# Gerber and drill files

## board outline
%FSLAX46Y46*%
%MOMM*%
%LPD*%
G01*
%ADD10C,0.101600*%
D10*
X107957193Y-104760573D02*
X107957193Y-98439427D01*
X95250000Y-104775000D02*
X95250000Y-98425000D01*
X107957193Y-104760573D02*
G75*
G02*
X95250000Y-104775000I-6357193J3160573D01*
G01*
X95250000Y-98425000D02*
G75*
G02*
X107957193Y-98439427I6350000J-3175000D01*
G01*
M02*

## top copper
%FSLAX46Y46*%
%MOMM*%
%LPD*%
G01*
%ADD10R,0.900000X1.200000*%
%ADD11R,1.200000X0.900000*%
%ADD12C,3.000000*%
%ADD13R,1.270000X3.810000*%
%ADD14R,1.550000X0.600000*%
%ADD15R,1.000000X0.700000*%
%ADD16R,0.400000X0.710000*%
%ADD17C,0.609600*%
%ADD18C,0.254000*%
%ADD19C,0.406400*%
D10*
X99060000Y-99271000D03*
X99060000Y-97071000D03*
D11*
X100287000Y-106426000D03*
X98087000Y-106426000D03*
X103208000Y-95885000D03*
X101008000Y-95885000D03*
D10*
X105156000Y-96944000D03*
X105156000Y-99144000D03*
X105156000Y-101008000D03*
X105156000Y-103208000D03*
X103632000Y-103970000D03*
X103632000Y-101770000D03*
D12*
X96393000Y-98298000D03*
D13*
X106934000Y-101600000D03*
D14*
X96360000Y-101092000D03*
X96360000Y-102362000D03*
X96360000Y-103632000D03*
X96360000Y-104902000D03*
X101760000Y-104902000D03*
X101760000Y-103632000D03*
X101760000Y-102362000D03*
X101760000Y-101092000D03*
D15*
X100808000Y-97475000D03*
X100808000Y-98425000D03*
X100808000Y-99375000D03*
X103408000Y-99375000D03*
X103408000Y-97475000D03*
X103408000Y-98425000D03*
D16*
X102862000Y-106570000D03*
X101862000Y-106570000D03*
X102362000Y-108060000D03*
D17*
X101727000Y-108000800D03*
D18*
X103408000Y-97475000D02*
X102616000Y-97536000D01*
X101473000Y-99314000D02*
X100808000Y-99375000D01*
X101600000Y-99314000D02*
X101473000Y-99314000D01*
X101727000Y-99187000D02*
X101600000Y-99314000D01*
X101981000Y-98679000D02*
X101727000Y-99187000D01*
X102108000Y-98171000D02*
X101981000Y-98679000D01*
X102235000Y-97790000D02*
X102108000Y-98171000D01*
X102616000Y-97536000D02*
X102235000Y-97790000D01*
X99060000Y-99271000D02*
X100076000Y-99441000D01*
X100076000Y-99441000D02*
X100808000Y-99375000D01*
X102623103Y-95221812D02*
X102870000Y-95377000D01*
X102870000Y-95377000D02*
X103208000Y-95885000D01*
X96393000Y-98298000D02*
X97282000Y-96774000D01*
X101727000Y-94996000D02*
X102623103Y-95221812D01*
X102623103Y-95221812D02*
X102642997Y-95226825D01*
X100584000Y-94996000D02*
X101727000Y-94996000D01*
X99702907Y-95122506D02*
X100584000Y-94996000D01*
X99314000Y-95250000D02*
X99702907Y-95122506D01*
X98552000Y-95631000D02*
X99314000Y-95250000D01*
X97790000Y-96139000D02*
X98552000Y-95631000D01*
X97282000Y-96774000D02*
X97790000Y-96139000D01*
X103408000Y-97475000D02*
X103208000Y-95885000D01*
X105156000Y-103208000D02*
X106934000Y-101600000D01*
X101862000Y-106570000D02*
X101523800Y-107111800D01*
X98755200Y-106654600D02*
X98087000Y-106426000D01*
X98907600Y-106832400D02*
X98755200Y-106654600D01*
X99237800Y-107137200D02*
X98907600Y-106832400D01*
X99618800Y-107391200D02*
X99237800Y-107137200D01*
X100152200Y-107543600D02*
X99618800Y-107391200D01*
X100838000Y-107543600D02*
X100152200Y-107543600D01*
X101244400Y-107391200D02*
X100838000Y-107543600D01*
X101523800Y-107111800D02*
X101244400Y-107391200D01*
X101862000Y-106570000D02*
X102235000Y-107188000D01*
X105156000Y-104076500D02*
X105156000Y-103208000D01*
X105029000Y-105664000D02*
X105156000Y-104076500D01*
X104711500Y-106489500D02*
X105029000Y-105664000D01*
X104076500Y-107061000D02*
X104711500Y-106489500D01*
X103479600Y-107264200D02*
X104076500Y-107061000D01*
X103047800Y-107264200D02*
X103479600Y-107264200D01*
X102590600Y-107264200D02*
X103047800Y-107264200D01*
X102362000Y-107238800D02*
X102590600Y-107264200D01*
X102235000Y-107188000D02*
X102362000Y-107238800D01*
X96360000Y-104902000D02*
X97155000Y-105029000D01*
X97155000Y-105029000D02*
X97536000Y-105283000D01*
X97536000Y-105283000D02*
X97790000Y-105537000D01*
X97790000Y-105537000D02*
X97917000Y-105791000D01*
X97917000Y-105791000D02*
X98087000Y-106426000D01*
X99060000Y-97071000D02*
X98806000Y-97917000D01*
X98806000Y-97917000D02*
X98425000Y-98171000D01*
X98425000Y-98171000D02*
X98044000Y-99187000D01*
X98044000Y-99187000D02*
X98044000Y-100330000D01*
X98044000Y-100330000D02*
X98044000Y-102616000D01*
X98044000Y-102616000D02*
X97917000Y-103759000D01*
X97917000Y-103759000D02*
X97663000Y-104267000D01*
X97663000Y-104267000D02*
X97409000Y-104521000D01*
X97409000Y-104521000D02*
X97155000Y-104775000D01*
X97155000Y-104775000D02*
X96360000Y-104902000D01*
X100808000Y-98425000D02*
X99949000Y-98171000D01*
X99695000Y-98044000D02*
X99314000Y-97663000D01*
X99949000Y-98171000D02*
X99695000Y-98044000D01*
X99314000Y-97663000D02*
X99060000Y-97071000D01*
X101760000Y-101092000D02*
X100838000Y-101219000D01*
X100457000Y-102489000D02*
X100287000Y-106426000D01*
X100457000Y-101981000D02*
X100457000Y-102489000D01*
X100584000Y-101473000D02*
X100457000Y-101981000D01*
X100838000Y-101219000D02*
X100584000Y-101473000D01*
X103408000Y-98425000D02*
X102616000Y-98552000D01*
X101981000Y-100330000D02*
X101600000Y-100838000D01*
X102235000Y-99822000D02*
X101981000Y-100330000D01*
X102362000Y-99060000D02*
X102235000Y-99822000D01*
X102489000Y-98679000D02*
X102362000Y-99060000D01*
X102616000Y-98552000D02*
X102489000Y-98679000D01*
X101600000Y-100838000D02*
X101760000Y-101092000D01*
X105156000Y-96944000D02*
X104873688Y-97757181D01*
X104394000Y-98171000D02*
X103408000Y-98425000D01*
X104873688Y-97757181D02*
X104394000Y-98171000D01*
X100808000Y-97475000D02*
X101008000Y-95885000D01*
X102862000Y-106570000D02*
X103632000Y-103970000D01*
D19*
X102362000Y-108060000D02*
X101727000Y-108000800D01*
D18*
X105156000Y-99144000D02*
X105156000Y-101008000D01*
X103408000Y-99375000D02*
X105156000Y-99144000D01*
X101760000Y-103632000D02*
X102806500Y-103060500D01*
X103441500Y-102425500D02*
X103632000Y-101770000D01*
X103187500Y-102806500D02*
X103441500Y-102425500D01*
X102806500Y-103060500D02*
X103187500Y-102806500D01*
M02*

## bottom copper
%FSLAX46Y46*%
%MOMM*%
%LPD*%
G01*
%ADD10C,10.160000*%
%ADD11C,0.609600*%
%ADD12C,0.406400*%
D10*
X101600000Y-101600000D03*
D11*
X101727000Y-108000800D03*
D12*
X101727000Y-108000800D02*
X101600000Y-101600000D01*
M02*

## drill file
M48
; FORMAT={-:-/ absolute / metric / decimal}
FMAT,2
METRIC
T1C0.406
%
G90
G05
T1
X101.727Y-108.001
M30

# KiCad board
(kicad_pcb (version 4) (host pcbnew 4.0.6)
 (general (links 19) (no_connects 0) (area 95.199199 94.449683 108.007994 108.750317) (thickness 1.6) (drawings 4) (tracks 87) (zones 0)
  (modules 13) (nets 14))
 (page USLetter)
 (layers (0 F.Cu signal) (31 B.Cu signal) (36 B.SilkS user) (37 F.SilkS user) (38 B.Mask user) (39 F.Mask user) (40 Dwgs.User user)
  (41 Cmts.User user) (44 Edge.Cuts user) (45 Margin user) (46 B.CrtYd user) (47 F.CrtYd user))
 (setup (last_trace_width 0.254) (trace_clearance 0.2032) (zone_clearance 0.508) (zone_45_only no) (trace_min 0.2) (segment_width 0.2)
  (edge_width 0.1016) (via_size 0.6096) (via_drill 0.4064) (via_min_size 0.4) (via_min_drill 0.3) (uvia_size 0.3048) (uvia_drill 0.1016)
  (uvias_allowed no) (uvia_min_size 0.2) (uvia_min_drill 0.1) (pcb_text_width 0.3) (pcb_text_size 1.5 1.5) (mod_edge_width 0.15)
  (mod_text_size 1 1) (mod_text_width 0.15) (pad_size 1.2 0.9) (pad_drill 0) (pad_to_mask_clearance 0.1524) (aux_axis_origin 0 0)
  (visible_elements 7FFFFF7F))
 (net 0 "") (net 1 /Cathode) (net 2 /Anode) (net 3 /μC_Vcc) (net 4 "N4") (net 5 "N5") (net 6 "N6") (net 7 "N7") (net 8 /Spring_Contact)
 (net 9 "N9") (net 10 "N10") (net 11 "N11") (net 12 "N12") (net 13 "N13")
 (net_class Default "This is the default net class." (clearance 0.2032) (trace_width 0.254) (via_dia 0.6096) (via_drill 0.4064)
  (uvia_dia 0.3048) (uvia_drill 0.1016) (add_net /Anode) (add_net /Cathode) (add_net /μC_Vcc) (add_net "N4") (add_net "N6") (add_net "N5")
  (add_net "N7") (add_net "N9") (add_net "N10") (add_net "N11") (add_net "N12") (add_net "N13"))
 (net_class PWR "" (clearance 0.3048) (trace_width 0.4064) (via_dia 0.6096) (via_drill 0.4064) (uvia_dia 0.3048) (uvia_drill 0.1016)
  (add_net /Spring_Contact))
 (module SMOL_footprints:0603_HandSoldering (layer F.Cu) (at 99.06 98.171 90)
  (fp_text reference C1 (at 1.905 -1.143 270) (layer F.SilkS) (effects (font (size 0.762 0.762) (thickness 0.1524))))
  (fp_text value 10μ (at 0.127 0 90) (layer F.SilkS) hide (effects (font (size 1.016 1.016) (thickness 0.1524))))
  (pad 1 smd rect (at -1.1 0 90) (size 1.2 0.9) (layers F.Cu F.Mask) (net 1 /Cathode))
  (pad 2 smd rect (at 1.1 0 90) (size 1.2 0.9) (layers F.Cu F.Mask) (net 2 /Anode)))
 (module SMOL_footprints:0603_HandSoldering (layer F.Cu) (at 99.187 106.426 180)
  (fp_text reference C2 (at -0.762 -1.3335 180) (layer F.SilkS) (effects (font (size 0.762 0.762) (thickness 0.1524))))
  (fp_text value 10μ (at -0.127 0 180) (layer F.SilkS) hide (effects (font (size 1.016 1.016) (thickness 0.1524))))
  (pad 1 smd rect (at -1.1 0 180) (size 1.2 0.9) (layers F.Cu F.Mask) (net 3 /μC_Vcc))
  (pad 2 smd rect (at 1.1 0 180) (size 1.2 0.9) (layers F.Cu F.Mask) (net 2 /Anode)))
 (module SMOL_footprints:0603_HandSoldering (layer F.Cu) (at 102.108 95.885 180)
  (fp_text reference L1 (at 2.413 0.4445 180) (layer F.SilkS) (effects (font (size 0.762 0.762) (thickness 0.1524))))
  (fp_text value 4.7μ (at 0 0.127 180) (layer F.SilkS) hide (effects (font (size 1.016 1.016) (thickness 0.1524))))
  (pad 1 smd rect (at -1.1 0 180) (size 1.2 0.9) (layers F.Cu F.Mask) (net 1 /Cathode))
  (pad 2 smd rect (at 1.1 0 180) (size 1.2 0.9) (layers F.Cu F.Mask) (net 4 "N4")))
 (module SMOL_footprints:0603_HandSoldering (layer F.Cu) (at 105.156 98.044 270)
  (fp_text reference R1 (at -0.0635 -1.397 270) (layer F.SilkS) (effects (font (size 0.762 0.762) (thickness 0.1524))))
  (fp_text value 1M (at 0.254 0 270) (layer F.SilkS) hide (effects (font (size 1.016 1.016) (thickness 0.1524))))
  (pad 1 smd rect (at -1.1 0 270) (size 1.2 0.9) (layers F.Cu F.Mask) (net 3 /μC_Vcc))
  (pad 2 smd rect (at 1.1 0 270) (size 1.2 0.9) (layers F.Cu F.Mask) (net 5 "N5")))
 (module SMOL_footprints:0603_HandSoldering (layer F.Cu) (at 105.156 102.108 270)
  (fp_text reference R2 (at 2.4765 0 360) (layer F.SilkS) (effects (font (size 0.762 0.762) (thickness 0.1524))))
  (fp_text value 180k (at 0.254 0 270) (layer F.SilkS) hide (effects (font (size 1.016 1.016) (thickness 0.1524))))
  (pad 1 smd rect (at -1.1 0 270) (size 1.2 0.9) (layers F.Cu F.Mask) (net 5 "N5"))
  (pad 2 smd rect (at 1.1 0 270) (size 1.2 0.9) (layers F.Cu F.Mask) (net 2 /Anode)))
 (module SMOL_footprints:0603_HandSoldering (layer F.Cu) (at 103.632 102.87 90)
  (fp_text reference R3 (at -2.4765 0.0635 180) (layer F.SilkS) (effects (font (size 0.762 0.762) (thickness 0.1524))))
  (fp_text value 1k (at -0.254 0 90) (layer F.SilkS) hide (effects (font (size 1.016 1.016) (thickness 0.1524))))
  (pad 1 smd rect (at -1.1 0 90) (size 1.2 0.9) (layers F.Cu F.Mask) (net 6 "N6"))
  (pad 2 smd rect (at 1.1 0 90) (size 1.2 0.9) (layers F.Cu F.Mask) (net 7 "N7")))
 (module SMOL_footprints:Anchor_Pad (layer F.Cu) (at 96.393 98.298)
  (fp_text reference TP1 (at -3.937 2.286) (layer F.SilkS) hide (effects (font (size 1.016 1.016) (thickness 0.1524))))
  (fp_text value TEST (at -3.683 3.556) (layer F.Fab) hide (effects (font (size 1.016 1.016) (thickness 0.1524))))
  (pad 1 smd circle (at 0 0) (size 3 3) (layers F.Cu F.Mask) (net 1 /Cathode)))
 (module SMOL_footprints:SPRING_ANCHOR (layer F.Cu) (at 106.934 101.6)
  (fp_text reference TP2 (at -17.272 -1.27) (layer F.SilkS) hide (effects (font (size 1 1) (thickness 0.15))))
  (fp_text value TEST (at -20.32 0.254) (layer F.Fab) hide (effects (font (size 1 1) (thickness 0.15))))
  (pad 1 smd rect (at 0 0) (size 1.27 3.81) (layers F.Cu F.Mask) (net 2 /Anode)))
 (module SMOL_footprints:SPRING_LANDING (layer B.Cu) (at 93.037 97.622)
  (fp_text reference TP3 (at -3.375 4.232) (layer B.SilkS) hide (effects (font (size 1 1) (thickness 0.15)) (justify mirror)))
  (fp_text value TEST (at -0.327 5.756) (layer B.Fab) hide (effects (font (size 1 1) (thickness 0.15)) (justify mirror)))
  (pad 1 smd circle (at 8.563 3.978) (size 10.16 10.16) (layers B.Cu B.Mask) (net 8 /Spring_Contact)))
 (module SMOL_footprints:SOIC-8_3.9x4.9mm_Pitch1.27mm (layer F.Cu) (at 99.06 102.997)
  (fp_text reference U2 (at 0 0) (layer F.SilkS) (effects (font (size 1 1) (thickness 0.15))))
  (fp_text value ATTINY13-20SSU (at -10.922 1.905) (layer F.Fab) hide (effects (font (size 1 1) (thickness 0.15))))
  (pad 1 smd rect (at -2.7 -1.905) (size 1.55 0.6) (layers F.Cu F.Mask) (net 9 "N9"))
  (pad 2 smd rect (at -2.7 -0.635) (size 1.55 0.6) (layers F.Cu F.Mask) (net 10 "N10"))
  (pad 3 smd rect (at -2.7 0.635) (size 1.55 0.6) (layers F.Cu F.Mask) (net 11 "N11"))
  (pad 4 smd rect (at -2.7 1.905) (size 1.55 0.6) (layers F.Cu F.Mask) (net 2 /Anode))
  (pad 5 smd rect (at 2.7 1.905) (size 1.55 0.6) (layers F.Cu F.Mask) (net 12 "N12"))
  (pad 6 smd rect (at 2.7 0.635) (size 1.55 0.6) (layers F.Cu F.Mask) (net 7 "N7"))
  (pad 7 smd rect (at 2.7 -0.635) (size 1.55 0.6) (layers F.Cu F.Mask) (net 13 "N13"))
  (pad 8 smd rect (at 2.7 -1.905) (size 1.55 0.6) (layers F.Cu F.Mask) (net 3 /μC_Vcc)))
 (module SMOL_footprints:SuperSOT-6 (layer F.Cu) (at 102.108 98.425)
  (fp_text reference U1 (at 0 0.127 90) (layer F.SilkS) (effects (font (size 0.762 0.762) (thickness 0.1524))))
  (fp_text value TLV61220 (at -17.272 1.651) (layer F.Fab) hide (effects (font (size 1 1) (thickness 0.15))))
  (pad 1 smd rect (at -1.3 -0.95) (size 1 0.7) (layers F.Cu F.Mask) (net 4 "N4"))
  (pad 2 smd rect (at -1.3 0) (size 1 0.7) (layers F.Cu F.Mask) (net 2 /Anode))
  (pad 3 smd rect (at -1.3 0.95) (size 1 0.7) (layers F.Cu F.Mask) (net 1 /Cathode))
  (pad 4 smd rect (at 1.3 0.95) (size 1 0.7) (layers F.Cu F.Mask) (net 5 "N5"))
  (pad 6 smd rect (at 1.3 -0.95) (size 1 0.7) (layers F.Cu F.Mask) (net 1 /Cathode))
  (pad 5 smd rect (at 1.3 0) (size 1 0.7) (layers F.Cu F.Mask) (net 3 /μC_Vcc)))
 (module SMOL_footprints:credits (layer B.Cu) (at 101.6 101.6 90)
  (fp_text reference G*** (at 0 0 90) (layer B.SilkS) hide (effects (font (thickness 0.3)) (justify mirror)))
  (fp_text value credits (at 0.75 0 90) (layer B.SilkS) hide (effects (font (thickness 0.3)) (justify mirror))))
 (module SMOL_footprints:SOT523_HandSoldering (layer F.Cu) (at 102.362 107.315 180)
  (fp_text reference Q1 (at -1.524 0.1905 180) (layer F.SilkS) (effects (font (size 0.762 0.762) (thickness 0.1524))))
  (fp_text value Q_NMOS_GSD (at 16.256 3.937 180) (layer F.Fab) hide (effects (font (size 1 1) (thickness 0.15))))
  (pad 1 smd rect (at -0.5 0.745 180) (size 0.4 0.71) (layers F.Cu F.Mask) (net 6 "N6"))
  (pad 2 smd rect (at 0.5 0.745 180) (size 0.4 0.71) (layers F.Cu F.Mask) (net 2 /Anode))
  (pad 3 smd rect (at 0 -0.745 180) (size 0.4 0.71) (layers F.Cu F.Mask) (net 8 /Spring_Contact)))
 (gr_line (start 107.957193 104.760573) (end 107.957193 98.439427) (angle 90) (layer Edge.Cuts) (width 0.1016))
 (gr_line (start 95.25 104.775) (end 95.25 98.425) (angle 90) (layer Edge.Cuts) (width 0.1016))
 (gr_arc (start 101.6 101.6) (end 95.25 104.775) (angle -127) (layer Edge.Cuts) (width 0.1016))
 (gr_arc (start 101.6 101.6) (end 95.25 98.425) (angle 127) (layer Edge.Cuts) (width 0.1016))
 (segment (start 103.408 97.475) (end 102.616 97.536) (width 0.254) (layer F.Cu) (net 1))
 (segment (start 101.473 99.314) (end 100.808 99.375) (width 0.254) (layer F.Cu) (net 1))
 (segment (start 101.6 99.314) (end 101.473 99.314) (width 0.254) (layer F.Cu) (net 1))
 (segment (start 101.727 99.187) (end 101.6 99.314) (width 0.254) (layer F.Cu) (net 1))
 (segment (start 101.981 98.679) (end 101.727 99.187) (width 0.254) (layer F.Cu) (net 1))
 (segment (start 102.108 98.171) (end 101.981 98.679) (width 0.254) (layer F.Cu) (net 1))
 (segment (start 102.235 97.79) (end 102.108 98.171) (width 0.254) (layer F.Cu) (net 1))
 (segment (start 102.616 97.536) (end 102.235 97.79) (width 0.254) (layer F.Cu) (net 1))
 (segment (start 99.06 99.271) (end 100.076 99.441) (width 0.254) (layer F.Cu) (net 1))
 (segment (start 100.076 99.441) (end 100.808 99.375) (width 0.254) (layer F.Cu) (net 1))
 (segment (start 102.623103 95.221812) (end 102.87 95.377) (width 0.254) (layer F.Cu) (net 1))
 (segment (start 102.87 95.377) (end 103.208 95.885) (width 0.254) (layer F.Cu) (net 1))
 (segment (start 96.393 98.298) (end 97.282 96.774) (width 0.254) (layer F.Cu) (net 1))
 (segment (start 101.727 94.996) (end 102.623103 95.221812) (width 0.254) (layer F.Cu) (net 1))
 (segment (start 102.623103 95.221812) (end 102.642997 95.226825) (width 0.254) (layer F.Cu) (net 1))
 (segment (start 100.584 94.996) (end 101.727 94.996) (width 0.254) (layer F.Cu) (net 1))
 (segment (start 99.702907 95.122506) (end 100.584 94.996) (width 0.254) (layer F.Cu) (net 1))
 (segment (start 99.314 95.25) (end 99.702907 95.122506) (width 0.254) (layer F.Cu) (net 1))
 (segment (start 98.552 95.631) (end 99.314 95.25) (width 0.254) (layer F.Cu) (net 1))
 (segment (start 97.79 96.139) (end 98.552 95.631) (width 0.254) (layer F.Cu) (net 1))
 (segment (start 97.282 96.774) (end 97.79 96.139) (width 0.254) (layer F.Cu) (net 1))
 (segment (start 103.408 97.475) (end 103.208 95.885) (width 0.254) (layer F.Cu) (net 1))
 (segment (start 105.156 103.208) (end 106.934 101.6) (width 0.254) (layer F.Cu) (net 2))
 (segment (start 101.862 106.57) (end 101.5238 107.1118) (width 0.254) (layer F.Cu) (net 2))
 (segment (start 98.7552 106.6546) (end 98.087 106.426) (width 0.254) (layer F.Cu) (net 2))
 (segment (start 98.9076 106.8324) (end 98.7552 106.6546) (width 0.254) (layer F.Cu) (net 2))
 (segment (start 99.2378 107.1372) (end 98.9076 106.8324) (width 0.254) (layer F.Cu) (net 2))
 (segment (start 99.6188 107.3912) (end 99.2378 107.1372) (width 0.254) (layer F.Cu) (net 2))
 (segment (start 100.1522 107.5436) (end 99.6188 107.3912) (width 0.254) (layer F.Cu) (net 2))
 (segment (start 100.838 107.5436) (end 100.1522 107.5436) (width 0.254) (layer F.Cu) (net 2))
 (segment (start 101.2444 107.3912) (end 100.838 107.5436) (width 0.254) (layer F.Cu) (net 2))
 (segment (start 101.5238 107.1118) (end 101.2444 107.3912) (width 0.254) (layer F.Cu) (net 2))
 (segment (start 101.862 106.57) (end 102.235 107.188) (width 0.254) (layer F.Cu) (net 2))
 (segment (start 105.156 104.0765) (end 105.156 103.208) (width 0.254) (layer F.Cu) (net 2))
 (segment (start 105.029 105.664) (end 105.156 104.0765) (width 0.254) (layer F.Cu) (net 2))
 (segment (start 104.7115 106.4895) (end 105.029 105.664) (width 0.254) (layer F.Cu) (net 2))
 (segment (start 104.0765 107.061) (end 104.7115 106.4895) (width 0.254) (layer F.Cu) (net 2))
 (segment (start 103.4796 107.2642) (end 104.0765 107.061) (width 0.254) (layer F.Cu) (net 2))
 (segment (start 103.0478 107.2642) (end 103.4796 107.2642) (width 0.254) (layer F.Cu) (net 2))
 (segment (start 102.5906 107.2642) (end 103.0478 107.2642) (width 0.254) (layer F.Cu) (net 2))
 (segment (start 102.362 107.2388) (end 102.5906 107.2642) (width 0.254) (layer F.Cu) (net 2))
 (segment (start 102.235 107.188) (end 102.362 107.2388) (width 0.254) (layer F.Cu) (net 2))
 (segment (start 96.36 104.902) (end 97.155 105.029) (width 0.254) (layer F.Cu) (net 2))
 (segment (start 97.155 105.029) (end 97.536 105.283) (width 0.254) (layer F.Cu) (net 2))
 (segment (start 97.536 105.283) (end 97.79 105.537) (width 0.254) (layer F.Cu) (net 2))
 (segment (start 97.79 105.537) (end 97.917 105.791) (width 0.254) (layer F.Cu) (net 2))
 (segment (start 97.917 105.791) (end 98.087 106.426) (width 0.254) (layer F.Cu) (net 2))
 (segment (start 99.06 97.071) (end 98.806 97.917) (width 0.254) (layer F.Cu) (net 2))
 (segment (start 98.806 97.917) (end 98.425 98.171) (width 0.254) (layer F.Cu) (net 2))
 (segment (start 98.425 98.171) (end 98.044 99.187) (width 0.254) (layer F.Cu) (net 2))
 (segment (start 98.044 99.187) (end 98.044 100.33) (width 0.254) (layer F.Cu) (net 2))
 (segment (start 98.044 100.33) (end 98.044 102.616) (width 0.254) (layer F.Cu) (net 2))
 (segment (start 98.044 102.616) (end 97.917 103.759) (width 0.254) (layer F.Cu) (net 2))
 (segment (start 97.917 103.759) (end 97.663 104.267) (width 0.254) (layer F.Cu) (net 2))
 (segment (start 97.663 104.267) (end 97.409 104.521) (width 0.254) (layer F.Cu) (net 2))
 (segment (start 97.409 104.521) (end 97.155 104.775) (width 0.254) (layer F.Cu) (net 2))
 (segment (start 97.155 104.775) (end 96.36 104.902) (width 0.254) (layer F.Cu) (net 2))
 (segment (start 100.808 98.425) (end 99.949 98.171) (width 0.254) (layer F.Cu) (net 2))
 (segment (start 99.695 98.044) (end 99.314 97.663) (width 0.254) (layer F.Cu) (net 2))
 (segment (start 99.949 98.171) (end 99.695 98.044) (width 0.254) (layer F.Cu) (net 2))
 (segment (start 99.314 97.663) (end 99.06 97.071) (width 0.254) (layer F.Cu) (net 2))
 (segment (start 101.76 101.092) (end 100.838 101.219) (width 0.254) (layer F.Cu) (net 3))
 (segment (start 100.457 102.489) (end 100.287 106.426) (width 0.254) (layer F.Cu) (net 3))
 (segment (start 100.457 101.981) (end 100.457 102.489) (width 0.254) (layer F.Cu) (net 3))
 (segment (start 100.584 101.473) (end 100.457 101.981) (width 0.254) (layer F.Cu) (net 3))
 (segment (start 100.838 101.219) (end 100.584 101.473) (width 0.254) (layer F.Cu) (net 3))
 (segment (start 103.408 98.425) (end 102.616 98.552) (width 0.254) (layer F.Cu) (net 3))
 (segment (start 101.981 100.33) (end 101.6 100.838) (width 0.254) (layer F.Cu) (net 3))
 (segment (start 102.235 99.822) (end 101.981 100.33) (width 0.254) (layer F.Cu) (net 3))
 (segment (start 102.362 99.06) (end 102.235 99.822) (width 0.254) (layer F.Cu) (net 3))
 (segment (start 102.489 98.679) (end 102.362 99.06) (width 0.254) (layer F.Cu) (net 3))
 (segment (start 102.616 98.552) (end 102.489 98.679) (width 0.254) (layer F.Cu) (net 3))
 (segment (start 101.6 100.838) (end 101.76 101.092) (width 0.254) (layer F.Cu) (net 3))
 (segment (start 105.156 96.944) (end 104.873688 97.757181) (width 0.254) (layer F.Cu) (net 3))
 (segment (start 104.394 98.171) (end 103.408 98.425) (width 0.254) (layer F.Cu) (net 3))
 (segment (start 104.873688 97.757181) (end 104.394 98.171) (width 0.254) (layer F.Cu) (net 3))
 (segment (start 100.808 97.475) (end 101.008 95.885) (width 0.254) (layer F.Cu) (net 4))
 (segment (start 102.862 106.57) (end 103.632 103.97) (width 0.254) (layer F.Cu) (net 6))
 (segment (start 102.362 108.06) (end 101.727 108.0008) (width 0.4064) (layer F.Cu) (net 8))
 (segment (start 101.727 108.0008) (end 101.6 101.6) (width 0.4064) (layer B.Cu) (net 8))
 (via (at 101.727 108.0008) (size 0.6096) (drill 0.4064) (layers F.Cu B.Cu) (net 8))
 (segment (start 105.156 99.144) (end 105.156 101.008) (width 0.254) (layer F.Cu) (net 5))
 (segment (start 103.408 99.375) (end 105.156 99.144) (width 0.254) (layer F.Cu) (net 5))
 (segment (start 101.76 103.632) (end 102.8065 103.0605) (width 0.254) (layer F.Cu) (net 7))
 (segment (start 103.4415 102.4255) (end 103.632 101.77) (width 0.254) (layer F.Cu) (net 7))
 (segment (start 103.1875 102.8065) (end 103.4415 102.4255) (width 0.254) (layer F.Cu) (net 7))
 (segment (start 102.8065 103.0605) (end 103.1875 102.8065) (width 0.254) (layer F.Cu) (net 7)))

